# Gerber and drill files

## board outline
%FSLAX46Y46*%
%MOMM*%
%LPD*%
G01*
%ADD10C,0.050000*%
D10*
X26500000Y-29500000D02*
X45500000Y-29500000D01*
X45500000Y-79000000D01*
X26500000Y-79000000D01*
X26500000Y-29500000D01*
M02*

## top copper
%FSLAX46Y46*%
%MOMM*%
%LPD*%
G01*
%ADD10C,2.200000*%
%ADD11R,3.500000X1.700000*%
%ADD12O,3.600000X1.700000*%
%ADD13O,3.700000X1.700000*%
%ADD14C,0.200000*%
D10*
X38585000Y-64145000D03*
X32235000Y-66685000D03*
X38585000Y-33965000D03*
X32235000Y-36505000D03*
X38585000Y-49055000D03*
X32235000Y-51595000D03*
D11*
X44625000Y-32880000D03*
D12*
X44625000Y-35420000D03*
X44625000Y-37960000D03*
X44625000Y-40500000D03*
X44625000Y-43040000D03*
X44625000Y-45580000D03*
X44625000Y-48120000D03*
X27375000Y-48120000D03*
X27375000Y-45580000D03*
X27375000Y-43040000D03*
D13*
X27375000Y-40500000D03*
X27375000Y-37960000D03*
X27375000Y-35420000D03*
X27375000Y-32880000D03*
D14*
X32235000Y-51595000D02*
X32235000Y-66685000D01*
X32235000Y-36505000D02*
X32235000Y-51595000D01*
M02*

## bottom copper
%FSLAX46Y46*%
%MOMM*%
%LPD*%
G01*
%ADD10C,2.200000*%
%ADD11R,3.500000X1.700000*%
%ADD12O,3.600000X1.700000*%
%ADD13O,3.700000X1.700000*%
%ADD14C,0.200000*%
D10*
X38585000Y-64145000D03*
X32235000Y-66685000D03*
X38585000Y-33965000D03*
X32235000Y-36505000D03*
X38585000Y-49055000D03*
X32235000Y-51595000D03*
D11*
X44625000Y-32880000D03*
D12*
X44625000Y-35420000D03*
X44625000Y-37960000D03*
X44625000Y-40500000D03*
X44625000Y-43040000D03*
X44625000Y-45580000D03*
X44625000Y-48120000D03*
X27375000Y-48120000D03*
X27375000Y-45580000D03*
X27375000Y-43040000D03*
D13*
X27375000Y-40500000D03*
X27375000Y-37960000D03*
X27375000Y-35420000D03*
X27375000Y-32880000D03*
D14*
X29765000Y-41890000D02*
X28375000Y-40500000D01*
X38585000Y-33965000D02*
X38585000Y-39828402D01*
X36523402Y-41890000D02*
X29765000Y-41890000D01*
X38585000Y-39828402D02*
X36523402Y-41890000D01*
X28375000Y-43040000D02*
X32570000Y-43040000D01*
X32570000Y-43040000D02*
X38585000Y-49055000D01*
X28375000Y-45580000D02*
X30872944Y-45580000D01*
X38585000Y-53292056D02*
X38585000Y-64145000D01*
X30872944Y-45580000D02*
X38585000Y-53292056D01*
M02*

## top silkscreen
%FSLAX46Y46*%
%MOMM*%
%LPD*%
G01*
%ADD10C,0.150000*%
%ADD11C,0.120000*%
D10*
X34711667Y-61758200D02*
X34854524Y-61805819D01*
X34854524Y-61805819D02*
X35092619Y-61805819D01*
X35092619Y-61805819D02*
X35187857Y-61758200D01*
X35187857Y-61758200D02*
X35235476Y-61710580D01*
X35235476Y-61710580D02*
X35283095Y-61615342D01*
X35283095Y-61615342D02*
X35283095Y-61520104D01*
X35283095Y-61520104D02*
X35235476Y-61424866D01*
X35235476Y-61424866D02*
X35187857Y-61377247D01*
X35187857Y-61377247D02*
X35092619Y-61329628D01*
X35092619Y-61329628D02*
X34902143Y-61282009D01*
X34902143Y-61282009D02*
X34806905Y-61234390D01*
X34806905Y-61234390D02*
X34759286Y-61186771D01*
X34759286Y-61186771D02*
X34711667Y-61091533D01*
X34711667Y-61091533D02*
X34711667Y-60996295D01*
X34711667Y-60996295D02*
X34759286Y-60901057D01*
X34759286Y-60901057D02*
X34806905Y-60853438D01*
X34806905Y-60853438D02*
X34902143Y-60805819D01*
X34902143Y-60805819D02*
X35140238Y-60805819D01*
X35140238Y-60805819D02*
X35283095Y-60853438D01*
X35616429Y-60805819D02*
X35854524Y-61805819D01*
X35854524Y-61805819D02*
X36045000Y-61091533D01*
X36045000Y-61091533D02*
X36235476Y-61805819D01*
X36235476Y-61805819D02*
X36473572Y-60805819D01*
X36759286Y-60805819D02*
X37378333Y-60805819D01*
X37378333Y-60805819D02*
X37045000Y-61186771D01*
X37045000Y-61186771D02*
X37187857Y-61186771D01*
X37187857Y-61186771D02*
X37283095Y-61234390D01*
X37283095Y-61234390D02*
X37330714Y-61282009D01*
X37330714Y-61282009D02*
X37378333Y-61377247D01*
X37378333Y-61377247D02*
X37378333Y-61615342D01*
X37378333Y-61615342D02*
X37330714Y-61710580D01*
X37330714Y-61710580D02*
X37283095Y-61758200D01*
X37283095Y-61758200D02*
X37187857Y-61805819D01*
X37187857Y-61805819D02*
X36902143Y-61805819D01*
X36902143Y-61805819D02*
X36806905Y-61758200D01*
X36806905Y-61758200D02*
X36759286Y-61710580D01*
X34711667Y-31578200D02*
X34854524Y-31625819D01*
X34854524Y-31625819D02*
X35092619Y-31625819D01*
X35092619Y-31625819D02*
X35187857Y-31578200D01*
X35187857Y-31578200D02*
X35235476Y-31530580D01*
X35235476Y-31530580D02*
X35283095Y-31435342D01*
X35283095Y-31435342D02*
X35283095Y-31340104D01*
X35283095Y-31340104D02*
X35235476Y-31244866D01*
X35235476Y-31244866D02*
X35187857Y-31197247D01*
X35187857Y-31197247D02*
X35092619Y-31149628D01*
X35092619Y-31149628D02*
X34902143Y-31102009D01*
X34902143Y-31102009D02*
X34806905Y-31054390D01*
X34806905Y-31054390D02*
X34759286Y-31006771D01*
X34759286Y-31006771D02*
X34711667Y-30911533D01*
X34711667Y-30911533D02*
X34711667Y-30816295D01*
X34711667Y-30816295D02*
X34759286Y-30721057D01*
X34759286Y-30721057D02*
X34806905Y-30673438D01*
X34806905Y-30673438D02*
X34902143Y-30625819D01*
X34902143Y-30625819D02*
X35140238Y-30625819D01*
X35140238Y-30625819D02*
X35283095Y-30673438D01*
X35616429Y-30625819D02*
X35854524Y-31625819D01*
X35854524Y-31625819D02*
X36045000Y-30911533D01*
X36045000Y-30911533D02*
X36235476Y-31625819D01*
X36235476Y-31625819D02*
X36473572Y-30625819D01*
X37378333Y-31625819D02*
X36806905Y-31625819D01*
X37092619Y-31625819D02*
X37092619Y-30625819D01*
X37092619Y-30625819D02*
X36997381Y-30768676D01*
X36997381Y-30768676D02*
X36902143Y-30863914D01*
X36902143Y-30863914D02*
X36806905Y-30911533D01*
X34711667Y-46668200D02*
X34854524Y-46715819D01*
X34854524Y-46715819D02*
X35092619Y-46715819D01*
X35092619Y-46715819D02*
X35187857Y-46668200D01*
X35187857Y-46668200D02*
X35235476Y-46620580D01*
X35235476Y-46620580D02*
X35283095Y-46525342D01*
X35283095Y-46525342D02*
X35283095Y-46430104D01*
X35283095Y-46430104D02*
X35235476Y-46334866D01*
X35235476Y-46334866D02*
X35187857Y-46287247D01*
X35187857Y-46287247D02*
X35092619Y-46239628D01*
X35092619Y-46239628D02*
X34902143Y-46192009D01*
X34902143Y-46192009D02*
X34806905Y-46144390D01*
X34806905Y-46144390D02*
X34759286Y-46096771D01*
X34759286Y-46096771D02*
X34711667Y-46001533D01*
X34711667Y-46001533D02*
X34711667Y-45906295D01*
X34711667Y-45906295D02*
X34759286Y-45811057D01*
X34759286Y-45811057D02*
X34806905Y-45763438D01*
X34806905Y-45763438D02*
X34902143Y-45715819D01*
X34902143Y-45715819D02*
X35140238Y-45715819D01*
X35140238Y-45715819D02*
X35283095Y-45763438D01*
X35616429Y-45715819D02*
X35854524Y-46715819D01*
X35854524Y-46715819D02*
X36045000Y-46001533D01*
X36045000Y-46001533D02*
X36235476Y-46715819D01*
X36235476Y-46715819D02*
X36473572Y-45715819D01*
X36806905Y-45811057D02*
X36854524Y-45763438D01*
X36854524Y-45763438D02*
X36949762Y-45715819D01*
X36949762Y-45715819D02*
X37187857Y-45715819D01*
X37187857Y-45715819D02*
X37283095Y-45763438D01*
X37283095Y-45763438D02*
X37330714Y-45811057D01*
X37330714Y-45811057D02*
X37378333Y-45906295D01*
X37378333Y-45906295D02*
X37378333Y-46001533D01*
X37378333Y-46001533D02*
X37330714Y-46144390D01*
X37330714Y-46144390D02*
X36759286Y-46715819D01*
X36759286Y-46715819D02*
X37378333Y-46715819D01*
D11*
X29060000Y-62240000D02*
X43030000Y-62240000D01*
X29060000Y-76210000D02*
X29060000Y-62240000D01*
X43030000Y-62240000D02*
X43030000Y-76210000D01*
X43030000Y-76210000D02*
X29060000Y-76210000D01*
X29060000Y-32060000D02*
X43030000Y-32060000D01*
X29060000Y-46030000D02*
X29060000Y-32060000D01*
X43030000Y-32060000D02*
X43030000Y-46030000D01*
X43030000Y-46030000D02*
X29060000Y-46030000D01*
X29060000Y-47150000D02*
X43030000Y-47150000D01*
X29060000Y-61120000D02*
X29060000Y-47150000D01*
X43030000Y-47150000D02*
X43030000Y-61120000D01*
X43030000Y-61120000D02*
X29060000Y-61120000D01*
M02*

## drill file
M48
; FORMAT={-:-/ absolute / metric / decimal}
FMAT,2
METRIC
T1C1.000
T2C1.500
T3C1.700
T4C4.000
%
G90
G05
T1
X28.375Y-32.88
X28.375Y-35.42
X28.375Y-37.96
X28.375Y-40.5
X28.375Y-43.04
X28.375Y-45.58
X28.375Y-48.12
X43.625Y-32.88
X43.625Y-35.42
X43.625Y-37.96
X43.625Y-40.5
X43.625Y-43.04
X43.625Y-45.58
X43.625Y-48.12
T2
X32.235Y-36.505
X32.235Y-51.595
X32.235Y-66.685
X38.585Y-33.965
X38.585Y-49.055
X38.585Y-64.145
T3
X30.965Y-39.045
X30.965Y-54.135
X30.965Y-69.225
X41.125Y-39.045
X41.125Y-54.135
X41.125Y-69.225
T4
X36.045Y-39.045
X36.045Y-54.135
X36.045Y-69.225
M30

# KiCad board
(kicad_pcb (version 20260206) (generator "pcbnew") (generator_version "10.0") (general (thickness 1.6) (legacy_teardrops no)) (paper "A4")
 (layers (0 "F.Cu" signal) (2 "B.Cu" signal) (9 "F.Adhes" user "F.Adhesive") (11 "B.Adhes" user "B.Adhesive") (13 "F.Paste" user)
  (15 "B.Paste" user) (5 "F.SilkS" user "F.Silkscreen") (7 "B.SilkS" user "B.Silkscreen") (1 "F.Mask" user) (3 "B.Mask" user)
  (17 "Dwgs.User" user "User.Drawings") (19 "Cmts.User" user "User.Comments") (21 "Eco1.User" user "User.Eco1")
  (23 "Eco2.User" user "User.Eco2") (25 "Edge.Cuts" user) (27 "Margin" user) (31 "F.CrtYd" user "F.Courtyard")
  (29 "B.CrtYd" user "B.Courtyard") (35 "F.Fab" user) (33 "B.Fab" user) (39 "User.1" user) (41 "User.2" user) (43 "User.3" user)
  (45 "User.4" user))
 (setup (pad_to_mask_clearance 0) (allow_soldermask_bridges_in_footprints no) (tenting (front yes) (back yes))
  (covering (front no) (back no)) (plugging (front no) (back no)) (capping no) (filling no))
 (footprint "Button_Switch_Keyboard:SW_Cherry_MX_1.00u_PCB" (layer "F.Cu") (at 38.585 64.145)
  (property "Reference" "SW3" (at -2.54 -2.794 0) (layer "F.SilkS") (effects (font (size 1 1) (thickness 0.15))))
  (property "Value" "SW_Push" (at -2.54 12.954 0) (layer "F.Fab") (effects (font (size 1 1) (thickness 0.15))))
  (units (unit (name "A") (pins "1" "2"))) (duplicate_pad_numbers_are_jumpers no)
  (fp_line (start -9.525 -1.905) (end 4.445 -1.905) (stroke (width 0.12) (type solid)) (layer "F.SilkS"))
  (fp_line (start -9.525 12.065) (end -9.525 -1.905) (stroke (width 0.12) (type solid)) (layer "F.SilkS"))
  (fp_line (start 4.445 -1.905) (end 4.445 12.065) (stroke (width 0.12) (type solid)) (layer "F.SilkS"))
  (fp_line (start 4.445 12.065) (end -9.525 12.065) (stroke (width 0.12) (type solid)) (layer "F.SilkS"))
  (pad "" np_thru_hole circle (at -7.62 5.08) (size 1.7 1.7) (drill 1.7) (layers "*.Cu" "*.Mask"))
  (pad "" np_thru_hole circle (at -2.54 5.08) (size 4 4) (drill 4) (layers "*.Cu" "*.Mask"))
  (pad "" np_thru_hole circle (at 2.54 5.08) (size 1.7 1.7) (drill 1.7) (layers "*.Cu" "*.Mask"))
  (pad "1" thru_hole circle (at 0 0) (size 2.2 2.2) (drill 1.5) (layers "*.Cu" "*.Mask") (remove_unused_layers no)
   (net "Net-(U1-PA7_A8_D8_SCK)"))
  (pad "2" thru_hole circle (at -6.35 2.54) (size 2.2 2.2) (drill 1.5) (layers "*.Cu" "*.Mask") (remove_unused_layers no) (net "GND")))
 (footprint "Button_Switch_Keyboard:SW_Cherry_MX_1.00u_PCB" (layer "F.Cu") (at 38.585 33.965)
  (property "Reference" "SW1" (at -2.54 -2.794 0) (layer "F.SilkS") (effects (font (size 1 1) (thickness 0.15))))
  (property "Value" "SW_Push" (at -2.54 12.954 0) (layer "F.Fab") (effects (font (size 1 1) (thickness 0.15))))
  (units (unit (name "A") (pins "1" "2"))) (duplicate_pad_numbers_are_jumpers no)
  (fp_line (start -9.525 -1.905) (end 4.445 -1.905) (stroke (width 0.12) (type solid)) (layer "F.SilkS"))
  (fp_line (start -9.525 12.065) (end -9.525 -1.905) (stroke (width 0.12) (type solid)) (layer "F.SilkS"))
  (fp_line (start 4.445 -1.905) (end 4.445 12.065) (stroke (width 0.12) (type solid)) (layer "F.SilkS"))
  (fp_line (start 4.445 12.065) (end -9.525 12.065) (stroke (width 0.12) (type solid)) (layer "F.SilkS"))
  (pad "" np_thru_hole circle (at -7.62 5.08) (size 1.7 1.7) (drill 1.7) (layers "*.Cu" "*.Mask"))
  (pad "" np_thru_hole circle (at -2.54 5.08) (size 4 4) (drill 4) (layers "*.Cu" "*.Mask"))
  (pad "" np_thru_hole circle (at 2.54 5.08) (size 1.7 1.7) (drill 1.7) (layers "*.Cu" "*.Mask"))
  (pad "1" thru_hole circle (at 0 0) (size 2.2 2.2) (drill 1.5) (layers "*.Cu" "*.Mask") (remove_unused_layers no)
   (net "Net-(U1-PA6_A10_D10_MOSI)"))
  (pad "2" thru_hole circle (at -6.35 2.54) (size 2.2 2.2) (drill 1.5) (layers "*.Cu" "*.Mask") (remove_unused_layers no) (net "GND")))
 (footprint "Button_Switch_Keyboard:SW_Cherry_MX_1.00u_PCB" (layer "F.Cu") (at 38.585 49.055)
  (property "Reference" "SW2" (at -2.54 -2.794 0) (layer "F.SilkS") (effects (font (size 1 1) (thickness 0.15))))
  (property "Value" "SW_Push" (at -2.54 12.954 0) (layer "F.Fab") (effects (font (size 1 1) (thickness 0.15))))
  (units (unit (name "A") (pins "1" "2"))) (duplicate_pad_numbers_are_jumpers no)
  (fp_line (start -9.525 -1.905) (end 4.445 -1.905) (stroke (width 0.12) (type solid)) (layer "F.SilkS"))
  (fp_line (start -9.525 12.065) (end -9.525 -1.905) (stroke (width 0.12) (type solid)) (layer "F.SilkS"))
  (fp_line (start 4.445 -1.905) (end 4.445 12.065) (stroke (width 0.12) (type solid)) (layer "F.SilkS"))
  (fp_line (start 4.445 12.065) (end -9.525 12.065) (stroke (width 0.12) (type solid)) (layer "F.SilkS"))
  (pad "" np_thru_hole circle (at -7.62 5.08) (size 1.7 1.7) (drill 1.7) (layers "*.Cu" "*.Mask"))
  (pad "" np_thru_hole circle (at -2.54 5.08) (size 4 4) (drill 4) (layers "*.Cu" "*.Mask"))
  (pad "" np_thru_hole circle (at 2.54 5.08) (size 1.7 1.7) (drill 1.7) (layers "*.Cu" "*.Mask"))
  (pad "1" thru_hole circle (at 0 0) (size 2.2 2.2) (drill 1.5) (layers "*.Cu" "*.Mask") (remove_unused_layers no)
   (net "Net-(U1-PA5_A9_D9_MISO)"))
  (pad "2" thru_hole circle (at -6.35 2.54) (size 2.2 2.2) (drill 1.5) (layers "*.Cu" "*.Mask") (remove_unused_layers no) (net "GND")))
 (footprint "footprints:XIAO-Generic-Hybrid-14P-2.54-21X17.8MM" (layer "B.Cu") (at 36 40.5 180)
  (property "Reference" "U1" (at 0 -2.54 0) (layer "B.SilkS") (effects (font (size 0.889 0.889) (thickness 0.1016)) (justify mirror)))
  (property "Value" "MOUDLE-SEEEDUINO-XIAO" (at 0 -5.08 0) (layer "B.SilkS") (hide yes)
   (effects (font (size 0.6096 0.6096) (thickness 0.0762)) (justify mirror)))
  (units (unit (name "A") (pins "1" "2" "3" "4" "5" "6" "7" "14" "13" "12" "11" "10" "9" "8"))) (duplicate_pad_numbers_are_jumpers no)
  (pad "1" thru_hole rect (at -7.625 7.62 180) (size 3.5 1.7) (drill 1 (offset -1 0)) (layers "*.Cu" "*.Mask") (remove_unused_layers no)
   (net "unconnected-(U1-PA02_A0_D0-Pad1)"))
  (pad "2" thru_hole oval (at -7.625 5.08 180) (size 3.6 1.7) (drill 1 (offset -1 0)) (layers "*.Cu" "*.Mask") (remove_unused_layers no)
   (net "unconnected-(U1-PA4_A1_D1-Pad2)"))
  (pad "3" thru_hole oval (at -7.625 2.54 180) (size 3.6 1.7) (drill 1 (offset -1 0)) (layers "*.Cu" "*.Mask") (remove_unused_layers no)
   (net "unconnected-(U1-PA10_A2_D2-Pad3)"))
  (pad "4" thru_hole oval (at -7.625 0 180) (size 3.6 1.7) (drill 1 (offset -1 0)) (layers "*.Cu" "*.Mask") (remove_unused_layers no)
   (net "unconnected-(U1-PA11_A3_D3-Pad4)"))
  (pad "5" thru_hole oval (at -7.625 -2.54 180) (size 3.6 1.7) (drill 1 (offset -1 0)) (layers "*.Cu" "*.Mask") (remove_unused_layers no)
   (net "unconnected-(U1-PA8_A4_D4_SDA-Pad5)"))
  (pad "6" thru_hole oval (at -7.625 -5.08) (size 3.6 1.7) (drill 1 (offset 1 0)) (layers "*.Cu" "*.Mask") (remove_unused_layers no)
   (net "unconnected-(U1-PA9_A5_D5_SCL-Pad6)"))
  (pad "7" thru_hole oval (at -7.625 -7.62 180) (size 3.6 1.7) (drill 1 (offset -1 0)) (layers "*.Cu" "*.Mask") (remove_unused_layers no)
   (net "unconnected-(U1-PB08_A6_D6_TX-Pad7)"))
  (pad "8" thru_hole oval (at 7.625 -7.62 180) (size 3.6 1.7) (drill 1 (offset 1 0)) (layers "*.Cu" "*.Mask") (remove_unused_layers no)
   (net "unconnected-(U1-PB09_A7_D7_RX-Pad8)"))
  (pad "9" thru_hole oval (at 7.625 -5.08 180) (size 3.6 1.7) (drill 1 (offset 1 0)) (layers "*.Cu" "*.Mask") (remove_unused_layers no)
   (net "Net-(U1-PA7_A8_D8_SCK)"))
  (pad "10" thru_hole oval (at 7.625 -2.54 180) (size 3.6 1.7) (drill 1 (offset 1 0)) (layers "*.Cu" "*.Mask") (remove_unused_layers no)
   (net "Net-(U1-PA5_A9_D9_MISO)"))
  (pad "11" thru_hole oval (at 7.625 0 180) (size 3.7 1.7) (drill 1 (offset 1 0)) (layers "*.Cu" "*.Mask") (remove_unused_layers no)
   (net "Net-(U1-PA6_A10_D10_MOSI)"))
  (pad "12" thru_hole oval (at 7.625 2.54 180) (size 3.7 1.7) (drill 1 (offset 1 0)) (layers "*.Cu" "*.Mask") (remove_unused_layers no)
   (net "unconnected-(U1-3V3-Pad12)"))
  (pad "13" thru_hole oval (at 7.625 5.08 180) (size 3.7 1.7) (drill 1 (offset 1 0)) (layers "*.Cu" "*.Mask") (remove_unused_layers no)
   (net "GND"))
  (pad "14" thru_hole oval (at 7.625 7.62 180) (size 3.7 1.7) (drill 1 (offset 1 0)) (layers "*.Cu" "*.Mask") (remove_unused_layers no)
   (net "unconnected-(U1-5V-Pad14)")))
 (gr_rect (start 26.5 29.5) (end 45.5 79) (stroke (width 0.05) (type default)) (fill no) (layer "Edge.Cuts"))
 (segment (start 32.235 51.595) (end 32.235 66.685) (width 0.2) (layer "F.Cu") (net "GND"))
 (segment (start 32.235 36.505) (end 32.235 51.595) (width 0.2) (layer "F.Cu") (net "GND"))
 (segment (start 29.765 41.89) (end 28.375 40.5) (width 0.2) (layer "B.Cu") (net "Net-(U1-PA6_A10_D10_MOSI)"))
 (segment (start 38.585 33.965) (end 38.585 39.828402) (width 0.2) (layer "B.Cu") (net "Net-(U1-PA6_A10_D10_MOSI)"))
 (segment (start 36.523402 41.89) (end 29.765 41.89) (width 0.2) (layer "B.Cu") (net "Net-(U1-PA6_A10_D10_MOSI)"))
 (segment (start 38.585 39.828402) (end 36.523402 41.89) (width 0.2) (layer "B.Cu") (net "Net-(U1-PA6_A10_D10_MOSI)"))
 (segment (start 28.375 43.04) (end 32.57 43.04) (width 0.2) (layer "B.Cu") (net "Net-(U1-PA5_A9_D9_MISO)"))
 (segment (start 32.57 43.04) (end 38.585 49.055) (width 0.2) (layer "B.Cu") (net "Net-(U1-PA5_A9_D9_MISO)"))
 (segment (start 28.375 45.58) (end 30.872944 45.58) (width 0.2) (layer "B.Cu") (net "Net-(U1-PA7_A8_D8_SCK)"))
 (segment (start 38.585 53.292056) (end 38.585 64.145) (width 0.2) (layer "B.Cu") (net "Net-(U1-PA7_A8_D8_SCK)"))
 (segment (start 30.872944 45.58) (end 38.585 53.292056) (width 0.2) (layer "B.Cu") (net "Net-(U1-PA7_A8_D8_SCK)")))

